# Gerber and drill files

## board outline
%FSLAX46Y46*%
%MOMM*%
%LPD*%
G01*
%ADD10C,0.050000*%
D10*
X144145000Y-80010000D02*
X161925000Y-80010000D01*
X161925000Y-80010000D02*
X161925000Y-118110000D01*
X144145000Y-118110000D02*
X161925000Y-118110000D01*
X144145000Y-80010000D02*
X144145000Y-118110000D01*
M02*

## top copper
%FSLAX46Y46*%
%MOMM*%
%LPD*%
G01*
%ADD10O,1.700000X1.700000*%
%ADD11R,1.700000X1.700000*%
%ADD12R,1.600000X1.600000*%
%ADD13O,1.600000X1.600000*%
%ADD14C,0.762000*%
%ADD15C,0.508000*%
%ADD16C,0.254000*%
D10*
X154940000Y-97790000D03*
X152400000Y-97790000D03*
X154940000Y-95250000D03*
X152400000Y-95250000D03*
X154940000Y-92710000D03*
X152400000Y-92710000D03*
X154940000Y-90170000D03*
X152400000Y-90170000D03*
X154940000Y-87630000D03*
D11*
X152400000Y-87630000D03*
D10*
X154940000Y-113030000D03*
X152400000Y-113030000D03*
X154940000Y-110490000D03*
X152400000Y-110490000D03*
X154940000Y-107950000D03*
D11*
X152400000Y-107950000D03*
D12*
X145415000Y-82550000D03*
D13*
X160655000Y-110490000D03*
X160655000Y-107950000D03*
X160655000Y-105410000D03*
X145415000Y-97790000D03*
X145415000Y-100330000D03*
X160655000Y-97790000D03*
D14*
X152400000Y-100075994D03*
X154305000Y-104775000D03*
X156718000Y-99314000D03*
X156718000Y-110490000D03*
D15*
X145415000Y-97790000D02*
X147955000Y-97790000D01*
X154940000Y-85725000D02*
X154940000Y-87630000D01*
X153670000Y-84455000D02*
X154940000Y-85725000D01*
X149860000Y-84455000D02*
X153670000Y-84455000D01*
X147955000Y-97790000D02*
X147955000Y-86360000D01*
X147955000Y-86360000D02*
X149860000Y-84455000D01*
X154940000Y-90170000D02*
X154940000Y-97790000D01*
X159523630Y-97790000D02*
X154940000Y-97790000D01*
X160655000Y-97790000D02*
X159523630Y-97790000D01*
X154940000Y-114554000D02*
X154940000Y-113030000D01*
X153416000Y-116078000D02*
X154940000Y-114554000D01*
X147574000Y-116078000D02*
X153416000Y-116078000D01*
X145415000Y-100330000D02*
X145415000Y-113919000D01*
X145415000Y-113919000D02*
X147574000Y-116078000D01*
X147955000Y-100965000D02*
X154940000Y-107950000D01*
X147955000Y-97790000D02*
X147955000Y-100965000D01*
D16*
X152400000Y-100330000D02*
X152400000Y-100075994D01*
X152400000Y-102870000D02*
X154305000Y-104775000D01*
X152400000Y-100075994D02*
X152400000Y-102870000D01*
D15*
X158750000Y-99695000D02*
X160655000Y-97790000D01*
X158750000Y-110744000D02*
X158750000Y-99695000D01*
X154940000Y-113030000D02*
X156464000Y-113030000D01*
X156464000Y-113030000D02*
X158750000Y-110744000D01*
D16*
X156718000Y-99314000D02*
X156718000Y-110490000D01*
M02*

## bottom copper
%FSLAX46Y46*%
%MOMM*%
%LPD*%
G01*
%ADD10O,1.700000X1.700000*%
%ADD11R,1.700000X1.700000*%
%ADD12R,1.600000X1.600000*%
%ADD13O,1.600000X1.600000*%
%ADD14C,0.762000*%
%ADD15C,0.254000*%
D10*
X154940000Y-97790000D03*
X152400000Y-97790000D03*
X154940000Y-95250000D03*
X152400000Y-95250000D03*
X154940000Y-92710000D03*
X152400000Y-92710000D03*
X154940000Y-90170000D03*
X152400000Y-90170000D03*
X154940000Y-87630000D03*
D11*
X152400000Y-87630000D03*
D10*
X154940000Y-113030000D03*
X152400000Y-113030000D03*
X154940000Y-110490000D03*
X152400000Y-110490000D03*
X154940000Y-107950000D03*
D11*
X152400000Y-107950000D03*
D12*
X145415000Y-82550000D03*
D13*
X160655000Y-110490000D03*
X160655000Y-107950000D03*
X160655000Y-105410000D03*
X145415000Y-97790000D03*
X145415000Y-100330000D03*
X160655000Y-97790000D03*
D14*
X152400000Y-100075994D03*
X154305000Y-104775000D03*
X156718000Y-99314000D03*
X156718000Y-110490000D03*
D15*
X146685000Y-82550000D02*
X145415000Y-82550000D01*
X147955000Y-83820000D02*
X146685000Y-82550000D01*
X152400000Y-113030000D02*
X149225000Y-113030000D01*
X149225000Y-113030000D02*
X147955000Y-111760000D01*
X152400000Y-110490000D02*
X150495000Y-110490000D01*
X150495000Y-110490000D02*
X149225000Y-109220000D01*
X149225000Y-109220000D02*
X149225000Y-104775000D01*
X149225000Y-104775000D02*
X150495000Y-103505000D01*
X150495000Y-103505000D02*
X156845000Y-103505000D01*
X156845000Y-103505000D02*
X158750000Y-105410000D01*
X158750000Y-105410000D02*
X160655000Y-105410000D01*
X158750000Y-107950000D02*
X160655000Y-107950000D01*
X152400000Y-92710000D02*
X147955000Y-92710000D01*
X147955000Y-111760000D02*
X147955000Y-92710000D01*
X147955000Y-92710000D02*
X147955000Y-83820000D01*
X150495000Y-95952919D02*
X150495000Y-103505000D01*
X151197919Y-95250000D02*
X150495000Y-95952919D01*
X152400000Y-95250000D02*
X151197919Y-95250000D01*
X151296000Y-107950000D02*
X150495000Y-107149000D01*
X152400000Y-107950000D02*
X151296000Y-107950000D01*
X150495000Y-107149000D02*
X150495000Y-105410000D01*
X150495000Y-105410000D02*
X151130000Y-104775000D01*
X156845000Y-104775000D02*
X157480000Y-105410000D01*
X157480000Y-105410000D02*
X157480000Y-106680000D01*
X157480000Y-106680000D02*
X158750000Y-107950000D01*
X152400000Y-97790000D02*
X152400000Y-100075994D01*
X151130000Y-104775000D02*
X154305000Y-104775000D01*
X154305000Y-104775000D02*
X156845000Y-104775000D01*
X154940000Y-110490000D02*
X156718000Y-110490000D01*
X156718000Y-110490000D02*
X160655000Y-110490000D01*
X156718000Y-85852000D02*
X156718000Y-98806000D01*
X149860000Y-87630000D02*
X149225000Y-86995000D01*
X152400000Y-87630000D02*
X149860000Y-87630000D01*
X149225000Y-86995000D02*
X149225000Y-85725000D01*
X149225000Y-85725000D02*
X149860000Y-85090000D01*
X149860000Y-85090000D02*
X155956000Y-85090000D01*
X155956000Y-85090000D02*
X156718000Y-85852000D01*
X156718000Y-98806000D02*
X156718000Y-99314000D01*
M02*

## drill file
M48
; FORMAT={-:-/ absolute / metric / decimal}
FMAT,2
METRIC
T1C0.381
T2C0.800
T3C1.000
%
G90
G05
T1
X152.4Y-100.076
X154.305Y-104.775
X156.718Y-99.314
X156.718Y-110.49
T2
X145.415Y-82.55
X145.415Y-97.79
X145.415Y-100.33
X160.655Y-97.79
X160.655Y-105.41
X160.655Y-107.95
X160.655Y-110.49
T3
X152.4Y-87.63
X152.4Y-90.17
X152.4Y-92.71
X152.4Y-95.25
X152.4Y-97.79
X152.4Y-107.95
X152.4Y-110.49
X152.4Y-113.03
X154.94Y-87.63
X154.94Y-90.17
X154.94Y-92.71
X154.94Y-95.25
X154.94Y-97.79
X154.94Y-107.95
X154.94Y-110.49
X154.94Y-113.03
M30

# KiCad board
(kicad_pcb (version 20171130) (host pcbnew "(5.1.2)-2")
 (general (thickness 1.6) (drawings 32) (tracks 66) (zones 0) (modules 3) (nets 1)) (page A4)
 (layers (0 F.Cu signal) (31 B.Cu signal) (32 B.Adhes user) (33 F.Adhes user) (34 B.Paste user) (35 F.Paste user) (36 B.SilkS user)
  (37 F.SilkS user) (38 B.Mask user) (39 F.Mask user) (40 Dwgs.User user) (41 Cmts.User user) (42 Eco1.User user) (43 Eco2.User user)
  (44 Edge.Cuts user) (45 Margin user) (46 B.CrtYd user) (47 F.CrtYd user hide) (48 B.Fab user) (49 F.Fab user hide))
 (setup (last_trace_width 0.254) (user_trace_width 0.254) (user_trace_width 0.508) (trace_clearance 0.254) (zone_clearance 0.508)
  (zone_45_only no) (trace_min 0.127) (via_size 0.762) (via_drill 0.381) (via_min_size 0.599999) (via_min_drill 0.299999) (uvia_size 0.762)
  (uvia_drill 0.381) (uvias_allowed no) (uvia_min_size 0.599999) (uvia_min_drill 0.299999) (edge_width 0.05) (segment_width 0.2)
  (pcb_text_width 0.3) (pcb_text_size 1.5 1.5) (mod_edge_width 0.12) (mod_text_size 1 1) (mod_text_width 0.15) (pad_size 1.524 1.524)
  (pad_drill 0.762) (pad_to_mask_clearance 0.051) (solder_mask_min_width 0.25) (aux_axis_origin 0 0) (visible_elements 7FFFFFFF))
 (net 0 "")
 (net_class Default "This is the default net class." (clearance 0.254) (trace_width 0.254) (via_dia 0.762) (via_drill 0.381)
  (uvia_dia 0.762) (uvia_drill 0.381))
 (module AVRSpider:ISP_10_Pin (layer F.Cu) (at 152.4 87.63)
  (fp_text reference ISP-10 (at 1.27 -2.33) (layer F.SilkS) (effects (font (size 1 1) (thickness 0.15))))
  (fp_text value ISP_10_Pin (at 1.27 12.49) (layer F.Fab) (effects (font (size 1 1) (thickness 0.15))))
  (pad 10 thru_hole oval (at 2.54 10.16) (size 1.7 1.7) (drill 1) (layers *.Cu *.Mask))
  (pad 9 thru_hole oval (at 0 10.16) (size 1.7 1.7) (drill 1) (layers *.Cu *.Mask))
  (pad 8 thru_hole oval (at 2.54 7.62) (size 1.7 1.7) (drill 1) (layers *.Cu *.Mask))
  (pad 7 thru_hole oval (at 0 7.62) (size 1.7 1.7) (drill 1) (layers *.Cu *.Mask))
  (pad 6 thru_hole oval (at 2.54 5.08) (size 1.7 1.7) (drill 1) (layers *.Cu *.Mask))
  (pad 5 thru_hole oval (at 0 5.08) (size 1.7 1.7) (drill 1) (layers *.Cu *.Mask))
  (pad 4 thru_hole oval (at 2.54 2.54) (size 1.7 1.7) (drill 1) (layers *.Cu *.Mask))
  (pad 3 thru_hole oval (at 0 2.54) (size 1.7 1.7) (drill 1) (layers *.Cu *.Mask))
  (pad 2 thru_hole oval (at 2.54 0) (size 1.7 1.7) (drill 1) (layers *.Cu *.Mask))
  (pad 1 thru_hole rect (at 0 0) (size 1.7 1.7) (drill 1) (layers *.Cu *.Mask)))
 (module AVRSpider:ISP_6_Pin (layer F.Cu) (at 152.4 107.95)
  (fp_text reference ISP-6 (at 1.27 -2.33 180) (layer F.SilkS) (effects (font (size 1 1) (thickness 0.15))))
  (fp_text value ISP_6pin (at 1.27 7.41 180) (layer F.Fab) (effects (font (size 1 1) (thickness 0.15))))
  (pad 6 thru_hole oval (at 2.54 5.08) (size 1.7 1.7) (drill 1) (layers *.Cu *.Mask))
  (pad 5 thru_hole oval (at 0 5.08) (size 1.7 1.7) (drill 1) (layers *.Cu *.Mask))
  (pad 4 thru_hole oval (at 2.54 2.54) (size 1.7 1.7) (drill 1) (layers *.Cu *.Mask))
  (pad 3 thru_hole oval (at 0 2.54) (size 1.7 1.7) (drill 1) (layers *.Cu *.Mask))
  (pad 2 thru_hole oval (at 2.54 0) (size 1.7 1.7) (drill 1) (layers *.Cu *.Mask))
  (pad 1 thru_hole rect (at 0 0) (size 1.7 1.7) (drill 1) (layers *.Cu *.Mask)))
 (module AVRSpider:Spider (layer F.Cu) (at 145.415 82.55)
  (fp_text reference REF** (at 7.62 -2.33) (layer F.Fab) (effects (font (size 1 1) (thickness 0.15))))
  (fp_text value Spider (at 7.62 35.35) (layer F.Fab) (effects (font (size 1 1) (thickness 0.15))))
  (pad 1 thru_hole rect (at 0 0) (size 1.6 1.6) (drill 0.8) (layers *.Cu *.Mask))
  (pad 17 thru_hole oval (at 15.24 27.94) (size 1.6 1.6) (drill 0.8) (layers *.Cu *.Mask))
  (pad 18 thru_hole oval (at 15.24 25.4) (size 1.6 1.6) (drill 0.8) (layers *.Cu *.Mask))
  (pad 19 thru_hole oval (at 15.24 22.86) (size 1.6 1.6) (drill 0.8) (layers *.Cu *.Mask))
  (pad 7 thru_hole oval (at 0 15.24) (size 1.6 1.6) (drill 0.8) (layers *.Cu *.Mask))
  (pad 8 thru_hole oval (at 0 17.78) (size 1.6 1.6) (drill 0.8) (layers *.Cu *.Mask))
  (pad 22 thru_hole oval (at 15.24 15.24) (size 1.6 1.6) (drill 0.8) (layers *.Cu *.Mask)))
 (gr_line (start 144.145 80.01) (end 161.925 80.01) (layer Edge.Cuts) (width 0.05))
 (gr_line (start 161.925 80.01) (end 161.925 118.11) (layer Edge.Cuts) (width 0.05))
 (gr_line (start 144.145 118.11) (end 161.925 118.11) (layer Edge.Cuts) (width 0.05))
 (gr_line (start 144.145 80.01) (end 144.145 118.11) (layer Edge.Cuts) (width 0.05))
 (segment (start 145.415 97.79) (end 147.955 97.79) (width 0.508) (layer F.Cu) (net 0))
 (segment (start 154.94 85.725) (end 154.94 87.63) (width 0.508) (layer F.Cu) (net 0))
 (segment (start 153.67 84.455) (end 154.94 85.725) (width 0.508) (layer F.Cu) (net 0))
 (segment (start 149.86 84.455) (end 153.67 84.455) (width 0.508) (layer F.Cu) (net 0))
 (segment (start 147.955 97.79) (end 147.955 86.36) (width 0.508) (layer F.Cu) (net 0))
 (segment (start 147.955 86.36) (end 149.86 84.455) (width 0.508) (layer F.Cu) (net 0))
 (segment (start 146.685 82.55) (end 145.415 82.55) (width 0.254) (layer B.Cu) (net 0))
 (segment (start 147.955 83.82) (end 146.685 82.55) (width 0.254) (layer B.Cu) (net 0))
 (segment (start 152.4 113.03) (end 149.225 113.03) (width 0.254) (layer B.Cu) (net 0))
 (segment (start 149.225 113.03) (end 147.955 111.76) (width 0.254) (layer B.Cu) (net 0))
 (segment (start 152.4 110.49) (end 150.495 110.49) (width 0.254) (layer B.Cu) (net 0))
 (segment (start 150.495 110.49) (end 149.225 109.22) (width 0.254) (layer B.Cu) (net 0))
 (segment (start 149.225 109.22) (end 149.225 104.775) (width 0.254) (layer B.Cu) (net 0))
 (segment (start 149.225 104.775) (end 150.495 103.505) (width 0.254) (layer B.Cu) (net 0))
 (segment (start 150.495 103.505) (end 156.845 103.505) (width 0.254) (layer B.Cu) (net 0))
 (segment (start 156.845 103.505) (end 158.75 105.41) (width 0.254) (layer B.Cu) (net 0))
 (segment (start 158.75 105.41) (end 160.655 105.41) (width 0.254) (layer B.Cu) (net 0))
 (segment (start 158.75 107.95) (end 160.655 107.95) (width 0.254) (layer B.Cu) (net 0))
 (segment (start 152.4 92.71) (end 147.955 92.71) (width 0.254) (layer B.Cu) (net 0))
 (segment (start 147.955 111.76) (end 147.955 92.71) (width 0.254) (layer B.Cu) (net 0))
 (segment (start 147.955 92.71) (end 147.955 83.82) (width 0.254) (layer B.Cu) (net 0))
 (segment (start 150.495 95.952919) (end 150.495 103.505) (width 0.254) (layer B.Cu) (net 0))
 (segment (start 151.197919 95.25) (end 150.495 95.952919) (width 0.254) (layer B.Cu) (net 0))
 (segment (start 152.4 95.25) (end 151.197919 95.25) (width 0.254) (layer B.Cu) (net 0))
 (segment (start 151.296 107.95) (end 150.495 107.149) (width 0.254) (layer B.Cu) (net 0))
 (segment (start 152.4 107.95) (end 151.296 107.95) (width 0.254) (layer B.Cu) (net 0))
 (segment (start 150.495 107.149) (end 150.495 105.41) (width 0.254) (layer B.Cu) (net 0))
 (segment (start 150.495 105.41) (end 151.13 104.775) (width 0.254) (layer B.Cu) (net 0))
 (segment (start 156.845 104.775) (end 157.48 105.41) (width 0.254) (layer B.Cu) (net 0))
 (segment (start 157.48 105.41) (end 157.48 106.68) (width 0.254) (layer B.Cu) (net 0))
 (segment (start 157.48 106.68) (end 158.75 107.95) (width 0.254) (layer B.Cu) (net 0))
 (segment (start 154.94 90.17) (end 154.94 97.79) (width 0.508) (layer F.Cu) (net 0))
 (segment (start 159.52363 97.79) (end 154.94 97.79) (width 0.508) (layer F.Cu) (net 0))
 (segment (start 160.655 97.79) (end 159.52363 97.79) (width 0.508) (layer F.Cu) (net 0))
 (segment (start 154.94 114.554) (end 154.94 113.03) (width 0.508) (layer F.Cu) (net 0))
 (segment (start 153.416 116.078) (end 154.94 114.554) (width 0.508) (layer F.Cu) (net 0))
 (segment (start 147.574 116.078) (end 153.416 116.078) (width 0.508) (layer F.Cu) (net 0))
 (segment (start 145.415 100.33) (end 145.415 113.919) (width 0.508) (layer F.Cu) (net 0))
 (segment (start 145.415 113.919) (end 147.574 116.078) (width 0.508) (layer F.Cu) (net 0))
 (segment (start 147.955 100.965) (end 154.94 107.95) (width 0.508) (layer F.Cu) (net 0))
 (segment (start 147.955 97.79) (end 147.955 100.965) (width 0.508) (layer F.Cu) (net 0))
 (via (at 152.4 100.075994) (size 0.762) (drill 0.381) (layers F.Cu B.Cu) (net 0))
 (segment (start 152.4 97.79) (end 152.4 100.075994) (width 0.254) (layer B.Cu) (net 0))
 (segment (start 152.4 100.33) (end 152.4 100.075994) (width 0.254) (layer F.Cu) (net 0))
 (via (at 154.305 104.775) (size 0.762) (drill 0.381) (layers F.Cu B.Cu) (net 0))
 (segment (start 152.4 102.87) (end 154.305 104.775) (width 0.254) (layer F.Cu) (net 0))
 (segment (start 152.4 100.075994) (end 152.4 102.87) (width 0.254) (layer F.Cu) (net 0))
 (segment (start 151.13 104.775) (end 154.305 104.775) (width 0.254) (layer B.Cu) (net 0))
 (segment (start 154.305 104.775) (end 156.845 104.775) (width 0.254) (layer B.Cu) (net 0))
 (segment (start 158.75 99.695) (end 160.655 97.79) (width 0.508) (layer F.Cu) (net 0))
 (segment (start 158.75 110.744) (end 158.75 99.695) (width 0.508) (layer F.Cu) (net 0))
 (segment (start 154.94 113.03) (end 156.464 113.03) (width 0.508) (layer F.Cu) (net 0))
 (segment (start 156.464 113.03) (end 158.75 110.744) (width 0.508) (layer F.Cu) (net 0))
 (segment (start 154.94 110.49) (end 156.718 110.49) (width 0.254) (layer B.Cu) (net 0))
 (segment (start 156.718 110.49) (end 160.655 110.49) (width 0.254) (layer B.Cu) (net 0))
 (segment (start 156.718 85.852) (end 156.718 98.806) (width 0.254) (layer B.Cu) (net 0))
 (segment (start 149.86 87.63) (end 149.225 86.995) (width 0.254) (layer B.Cu) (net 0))
 (segment (start 152.4 87.63) (end 149.86 87.63) (width 0.254) (layer B.Cu) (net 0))
 (segment (start 149.225 86.995) (end 149.225 85.725) (width 0.254) (layer B.Cu) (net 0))
 (segment (start 149.225 85.725) (end 149.86 85.09) (width 0.254) (layer B.Cu) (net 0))
 (segment (start 149.86 85.09) (end 155.956 85.09) (width 0.254) (layer B.Cu) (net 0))
 (segment (start 155.956 85.09) (end 156.718 85.852) (width 0.254) (layer B.Cu) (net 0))
 (via (at 156.718 99.314) (size 0.762) (drill 0.381) (layers F.Cu B.Cu) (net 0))
 (segment (start 156.718 98.806) (end 156.718 99.314) (width 0.254) (layer B.Cu) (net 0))
 (via (at 156.718 110.49) (size 0.762) (drill 0.381) (layers F.Cu B.Cu) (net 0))
 (segment (start 156.718 99.314) (end 156.718 110.49) (width 0.254) (layer F.Cu) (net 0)))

